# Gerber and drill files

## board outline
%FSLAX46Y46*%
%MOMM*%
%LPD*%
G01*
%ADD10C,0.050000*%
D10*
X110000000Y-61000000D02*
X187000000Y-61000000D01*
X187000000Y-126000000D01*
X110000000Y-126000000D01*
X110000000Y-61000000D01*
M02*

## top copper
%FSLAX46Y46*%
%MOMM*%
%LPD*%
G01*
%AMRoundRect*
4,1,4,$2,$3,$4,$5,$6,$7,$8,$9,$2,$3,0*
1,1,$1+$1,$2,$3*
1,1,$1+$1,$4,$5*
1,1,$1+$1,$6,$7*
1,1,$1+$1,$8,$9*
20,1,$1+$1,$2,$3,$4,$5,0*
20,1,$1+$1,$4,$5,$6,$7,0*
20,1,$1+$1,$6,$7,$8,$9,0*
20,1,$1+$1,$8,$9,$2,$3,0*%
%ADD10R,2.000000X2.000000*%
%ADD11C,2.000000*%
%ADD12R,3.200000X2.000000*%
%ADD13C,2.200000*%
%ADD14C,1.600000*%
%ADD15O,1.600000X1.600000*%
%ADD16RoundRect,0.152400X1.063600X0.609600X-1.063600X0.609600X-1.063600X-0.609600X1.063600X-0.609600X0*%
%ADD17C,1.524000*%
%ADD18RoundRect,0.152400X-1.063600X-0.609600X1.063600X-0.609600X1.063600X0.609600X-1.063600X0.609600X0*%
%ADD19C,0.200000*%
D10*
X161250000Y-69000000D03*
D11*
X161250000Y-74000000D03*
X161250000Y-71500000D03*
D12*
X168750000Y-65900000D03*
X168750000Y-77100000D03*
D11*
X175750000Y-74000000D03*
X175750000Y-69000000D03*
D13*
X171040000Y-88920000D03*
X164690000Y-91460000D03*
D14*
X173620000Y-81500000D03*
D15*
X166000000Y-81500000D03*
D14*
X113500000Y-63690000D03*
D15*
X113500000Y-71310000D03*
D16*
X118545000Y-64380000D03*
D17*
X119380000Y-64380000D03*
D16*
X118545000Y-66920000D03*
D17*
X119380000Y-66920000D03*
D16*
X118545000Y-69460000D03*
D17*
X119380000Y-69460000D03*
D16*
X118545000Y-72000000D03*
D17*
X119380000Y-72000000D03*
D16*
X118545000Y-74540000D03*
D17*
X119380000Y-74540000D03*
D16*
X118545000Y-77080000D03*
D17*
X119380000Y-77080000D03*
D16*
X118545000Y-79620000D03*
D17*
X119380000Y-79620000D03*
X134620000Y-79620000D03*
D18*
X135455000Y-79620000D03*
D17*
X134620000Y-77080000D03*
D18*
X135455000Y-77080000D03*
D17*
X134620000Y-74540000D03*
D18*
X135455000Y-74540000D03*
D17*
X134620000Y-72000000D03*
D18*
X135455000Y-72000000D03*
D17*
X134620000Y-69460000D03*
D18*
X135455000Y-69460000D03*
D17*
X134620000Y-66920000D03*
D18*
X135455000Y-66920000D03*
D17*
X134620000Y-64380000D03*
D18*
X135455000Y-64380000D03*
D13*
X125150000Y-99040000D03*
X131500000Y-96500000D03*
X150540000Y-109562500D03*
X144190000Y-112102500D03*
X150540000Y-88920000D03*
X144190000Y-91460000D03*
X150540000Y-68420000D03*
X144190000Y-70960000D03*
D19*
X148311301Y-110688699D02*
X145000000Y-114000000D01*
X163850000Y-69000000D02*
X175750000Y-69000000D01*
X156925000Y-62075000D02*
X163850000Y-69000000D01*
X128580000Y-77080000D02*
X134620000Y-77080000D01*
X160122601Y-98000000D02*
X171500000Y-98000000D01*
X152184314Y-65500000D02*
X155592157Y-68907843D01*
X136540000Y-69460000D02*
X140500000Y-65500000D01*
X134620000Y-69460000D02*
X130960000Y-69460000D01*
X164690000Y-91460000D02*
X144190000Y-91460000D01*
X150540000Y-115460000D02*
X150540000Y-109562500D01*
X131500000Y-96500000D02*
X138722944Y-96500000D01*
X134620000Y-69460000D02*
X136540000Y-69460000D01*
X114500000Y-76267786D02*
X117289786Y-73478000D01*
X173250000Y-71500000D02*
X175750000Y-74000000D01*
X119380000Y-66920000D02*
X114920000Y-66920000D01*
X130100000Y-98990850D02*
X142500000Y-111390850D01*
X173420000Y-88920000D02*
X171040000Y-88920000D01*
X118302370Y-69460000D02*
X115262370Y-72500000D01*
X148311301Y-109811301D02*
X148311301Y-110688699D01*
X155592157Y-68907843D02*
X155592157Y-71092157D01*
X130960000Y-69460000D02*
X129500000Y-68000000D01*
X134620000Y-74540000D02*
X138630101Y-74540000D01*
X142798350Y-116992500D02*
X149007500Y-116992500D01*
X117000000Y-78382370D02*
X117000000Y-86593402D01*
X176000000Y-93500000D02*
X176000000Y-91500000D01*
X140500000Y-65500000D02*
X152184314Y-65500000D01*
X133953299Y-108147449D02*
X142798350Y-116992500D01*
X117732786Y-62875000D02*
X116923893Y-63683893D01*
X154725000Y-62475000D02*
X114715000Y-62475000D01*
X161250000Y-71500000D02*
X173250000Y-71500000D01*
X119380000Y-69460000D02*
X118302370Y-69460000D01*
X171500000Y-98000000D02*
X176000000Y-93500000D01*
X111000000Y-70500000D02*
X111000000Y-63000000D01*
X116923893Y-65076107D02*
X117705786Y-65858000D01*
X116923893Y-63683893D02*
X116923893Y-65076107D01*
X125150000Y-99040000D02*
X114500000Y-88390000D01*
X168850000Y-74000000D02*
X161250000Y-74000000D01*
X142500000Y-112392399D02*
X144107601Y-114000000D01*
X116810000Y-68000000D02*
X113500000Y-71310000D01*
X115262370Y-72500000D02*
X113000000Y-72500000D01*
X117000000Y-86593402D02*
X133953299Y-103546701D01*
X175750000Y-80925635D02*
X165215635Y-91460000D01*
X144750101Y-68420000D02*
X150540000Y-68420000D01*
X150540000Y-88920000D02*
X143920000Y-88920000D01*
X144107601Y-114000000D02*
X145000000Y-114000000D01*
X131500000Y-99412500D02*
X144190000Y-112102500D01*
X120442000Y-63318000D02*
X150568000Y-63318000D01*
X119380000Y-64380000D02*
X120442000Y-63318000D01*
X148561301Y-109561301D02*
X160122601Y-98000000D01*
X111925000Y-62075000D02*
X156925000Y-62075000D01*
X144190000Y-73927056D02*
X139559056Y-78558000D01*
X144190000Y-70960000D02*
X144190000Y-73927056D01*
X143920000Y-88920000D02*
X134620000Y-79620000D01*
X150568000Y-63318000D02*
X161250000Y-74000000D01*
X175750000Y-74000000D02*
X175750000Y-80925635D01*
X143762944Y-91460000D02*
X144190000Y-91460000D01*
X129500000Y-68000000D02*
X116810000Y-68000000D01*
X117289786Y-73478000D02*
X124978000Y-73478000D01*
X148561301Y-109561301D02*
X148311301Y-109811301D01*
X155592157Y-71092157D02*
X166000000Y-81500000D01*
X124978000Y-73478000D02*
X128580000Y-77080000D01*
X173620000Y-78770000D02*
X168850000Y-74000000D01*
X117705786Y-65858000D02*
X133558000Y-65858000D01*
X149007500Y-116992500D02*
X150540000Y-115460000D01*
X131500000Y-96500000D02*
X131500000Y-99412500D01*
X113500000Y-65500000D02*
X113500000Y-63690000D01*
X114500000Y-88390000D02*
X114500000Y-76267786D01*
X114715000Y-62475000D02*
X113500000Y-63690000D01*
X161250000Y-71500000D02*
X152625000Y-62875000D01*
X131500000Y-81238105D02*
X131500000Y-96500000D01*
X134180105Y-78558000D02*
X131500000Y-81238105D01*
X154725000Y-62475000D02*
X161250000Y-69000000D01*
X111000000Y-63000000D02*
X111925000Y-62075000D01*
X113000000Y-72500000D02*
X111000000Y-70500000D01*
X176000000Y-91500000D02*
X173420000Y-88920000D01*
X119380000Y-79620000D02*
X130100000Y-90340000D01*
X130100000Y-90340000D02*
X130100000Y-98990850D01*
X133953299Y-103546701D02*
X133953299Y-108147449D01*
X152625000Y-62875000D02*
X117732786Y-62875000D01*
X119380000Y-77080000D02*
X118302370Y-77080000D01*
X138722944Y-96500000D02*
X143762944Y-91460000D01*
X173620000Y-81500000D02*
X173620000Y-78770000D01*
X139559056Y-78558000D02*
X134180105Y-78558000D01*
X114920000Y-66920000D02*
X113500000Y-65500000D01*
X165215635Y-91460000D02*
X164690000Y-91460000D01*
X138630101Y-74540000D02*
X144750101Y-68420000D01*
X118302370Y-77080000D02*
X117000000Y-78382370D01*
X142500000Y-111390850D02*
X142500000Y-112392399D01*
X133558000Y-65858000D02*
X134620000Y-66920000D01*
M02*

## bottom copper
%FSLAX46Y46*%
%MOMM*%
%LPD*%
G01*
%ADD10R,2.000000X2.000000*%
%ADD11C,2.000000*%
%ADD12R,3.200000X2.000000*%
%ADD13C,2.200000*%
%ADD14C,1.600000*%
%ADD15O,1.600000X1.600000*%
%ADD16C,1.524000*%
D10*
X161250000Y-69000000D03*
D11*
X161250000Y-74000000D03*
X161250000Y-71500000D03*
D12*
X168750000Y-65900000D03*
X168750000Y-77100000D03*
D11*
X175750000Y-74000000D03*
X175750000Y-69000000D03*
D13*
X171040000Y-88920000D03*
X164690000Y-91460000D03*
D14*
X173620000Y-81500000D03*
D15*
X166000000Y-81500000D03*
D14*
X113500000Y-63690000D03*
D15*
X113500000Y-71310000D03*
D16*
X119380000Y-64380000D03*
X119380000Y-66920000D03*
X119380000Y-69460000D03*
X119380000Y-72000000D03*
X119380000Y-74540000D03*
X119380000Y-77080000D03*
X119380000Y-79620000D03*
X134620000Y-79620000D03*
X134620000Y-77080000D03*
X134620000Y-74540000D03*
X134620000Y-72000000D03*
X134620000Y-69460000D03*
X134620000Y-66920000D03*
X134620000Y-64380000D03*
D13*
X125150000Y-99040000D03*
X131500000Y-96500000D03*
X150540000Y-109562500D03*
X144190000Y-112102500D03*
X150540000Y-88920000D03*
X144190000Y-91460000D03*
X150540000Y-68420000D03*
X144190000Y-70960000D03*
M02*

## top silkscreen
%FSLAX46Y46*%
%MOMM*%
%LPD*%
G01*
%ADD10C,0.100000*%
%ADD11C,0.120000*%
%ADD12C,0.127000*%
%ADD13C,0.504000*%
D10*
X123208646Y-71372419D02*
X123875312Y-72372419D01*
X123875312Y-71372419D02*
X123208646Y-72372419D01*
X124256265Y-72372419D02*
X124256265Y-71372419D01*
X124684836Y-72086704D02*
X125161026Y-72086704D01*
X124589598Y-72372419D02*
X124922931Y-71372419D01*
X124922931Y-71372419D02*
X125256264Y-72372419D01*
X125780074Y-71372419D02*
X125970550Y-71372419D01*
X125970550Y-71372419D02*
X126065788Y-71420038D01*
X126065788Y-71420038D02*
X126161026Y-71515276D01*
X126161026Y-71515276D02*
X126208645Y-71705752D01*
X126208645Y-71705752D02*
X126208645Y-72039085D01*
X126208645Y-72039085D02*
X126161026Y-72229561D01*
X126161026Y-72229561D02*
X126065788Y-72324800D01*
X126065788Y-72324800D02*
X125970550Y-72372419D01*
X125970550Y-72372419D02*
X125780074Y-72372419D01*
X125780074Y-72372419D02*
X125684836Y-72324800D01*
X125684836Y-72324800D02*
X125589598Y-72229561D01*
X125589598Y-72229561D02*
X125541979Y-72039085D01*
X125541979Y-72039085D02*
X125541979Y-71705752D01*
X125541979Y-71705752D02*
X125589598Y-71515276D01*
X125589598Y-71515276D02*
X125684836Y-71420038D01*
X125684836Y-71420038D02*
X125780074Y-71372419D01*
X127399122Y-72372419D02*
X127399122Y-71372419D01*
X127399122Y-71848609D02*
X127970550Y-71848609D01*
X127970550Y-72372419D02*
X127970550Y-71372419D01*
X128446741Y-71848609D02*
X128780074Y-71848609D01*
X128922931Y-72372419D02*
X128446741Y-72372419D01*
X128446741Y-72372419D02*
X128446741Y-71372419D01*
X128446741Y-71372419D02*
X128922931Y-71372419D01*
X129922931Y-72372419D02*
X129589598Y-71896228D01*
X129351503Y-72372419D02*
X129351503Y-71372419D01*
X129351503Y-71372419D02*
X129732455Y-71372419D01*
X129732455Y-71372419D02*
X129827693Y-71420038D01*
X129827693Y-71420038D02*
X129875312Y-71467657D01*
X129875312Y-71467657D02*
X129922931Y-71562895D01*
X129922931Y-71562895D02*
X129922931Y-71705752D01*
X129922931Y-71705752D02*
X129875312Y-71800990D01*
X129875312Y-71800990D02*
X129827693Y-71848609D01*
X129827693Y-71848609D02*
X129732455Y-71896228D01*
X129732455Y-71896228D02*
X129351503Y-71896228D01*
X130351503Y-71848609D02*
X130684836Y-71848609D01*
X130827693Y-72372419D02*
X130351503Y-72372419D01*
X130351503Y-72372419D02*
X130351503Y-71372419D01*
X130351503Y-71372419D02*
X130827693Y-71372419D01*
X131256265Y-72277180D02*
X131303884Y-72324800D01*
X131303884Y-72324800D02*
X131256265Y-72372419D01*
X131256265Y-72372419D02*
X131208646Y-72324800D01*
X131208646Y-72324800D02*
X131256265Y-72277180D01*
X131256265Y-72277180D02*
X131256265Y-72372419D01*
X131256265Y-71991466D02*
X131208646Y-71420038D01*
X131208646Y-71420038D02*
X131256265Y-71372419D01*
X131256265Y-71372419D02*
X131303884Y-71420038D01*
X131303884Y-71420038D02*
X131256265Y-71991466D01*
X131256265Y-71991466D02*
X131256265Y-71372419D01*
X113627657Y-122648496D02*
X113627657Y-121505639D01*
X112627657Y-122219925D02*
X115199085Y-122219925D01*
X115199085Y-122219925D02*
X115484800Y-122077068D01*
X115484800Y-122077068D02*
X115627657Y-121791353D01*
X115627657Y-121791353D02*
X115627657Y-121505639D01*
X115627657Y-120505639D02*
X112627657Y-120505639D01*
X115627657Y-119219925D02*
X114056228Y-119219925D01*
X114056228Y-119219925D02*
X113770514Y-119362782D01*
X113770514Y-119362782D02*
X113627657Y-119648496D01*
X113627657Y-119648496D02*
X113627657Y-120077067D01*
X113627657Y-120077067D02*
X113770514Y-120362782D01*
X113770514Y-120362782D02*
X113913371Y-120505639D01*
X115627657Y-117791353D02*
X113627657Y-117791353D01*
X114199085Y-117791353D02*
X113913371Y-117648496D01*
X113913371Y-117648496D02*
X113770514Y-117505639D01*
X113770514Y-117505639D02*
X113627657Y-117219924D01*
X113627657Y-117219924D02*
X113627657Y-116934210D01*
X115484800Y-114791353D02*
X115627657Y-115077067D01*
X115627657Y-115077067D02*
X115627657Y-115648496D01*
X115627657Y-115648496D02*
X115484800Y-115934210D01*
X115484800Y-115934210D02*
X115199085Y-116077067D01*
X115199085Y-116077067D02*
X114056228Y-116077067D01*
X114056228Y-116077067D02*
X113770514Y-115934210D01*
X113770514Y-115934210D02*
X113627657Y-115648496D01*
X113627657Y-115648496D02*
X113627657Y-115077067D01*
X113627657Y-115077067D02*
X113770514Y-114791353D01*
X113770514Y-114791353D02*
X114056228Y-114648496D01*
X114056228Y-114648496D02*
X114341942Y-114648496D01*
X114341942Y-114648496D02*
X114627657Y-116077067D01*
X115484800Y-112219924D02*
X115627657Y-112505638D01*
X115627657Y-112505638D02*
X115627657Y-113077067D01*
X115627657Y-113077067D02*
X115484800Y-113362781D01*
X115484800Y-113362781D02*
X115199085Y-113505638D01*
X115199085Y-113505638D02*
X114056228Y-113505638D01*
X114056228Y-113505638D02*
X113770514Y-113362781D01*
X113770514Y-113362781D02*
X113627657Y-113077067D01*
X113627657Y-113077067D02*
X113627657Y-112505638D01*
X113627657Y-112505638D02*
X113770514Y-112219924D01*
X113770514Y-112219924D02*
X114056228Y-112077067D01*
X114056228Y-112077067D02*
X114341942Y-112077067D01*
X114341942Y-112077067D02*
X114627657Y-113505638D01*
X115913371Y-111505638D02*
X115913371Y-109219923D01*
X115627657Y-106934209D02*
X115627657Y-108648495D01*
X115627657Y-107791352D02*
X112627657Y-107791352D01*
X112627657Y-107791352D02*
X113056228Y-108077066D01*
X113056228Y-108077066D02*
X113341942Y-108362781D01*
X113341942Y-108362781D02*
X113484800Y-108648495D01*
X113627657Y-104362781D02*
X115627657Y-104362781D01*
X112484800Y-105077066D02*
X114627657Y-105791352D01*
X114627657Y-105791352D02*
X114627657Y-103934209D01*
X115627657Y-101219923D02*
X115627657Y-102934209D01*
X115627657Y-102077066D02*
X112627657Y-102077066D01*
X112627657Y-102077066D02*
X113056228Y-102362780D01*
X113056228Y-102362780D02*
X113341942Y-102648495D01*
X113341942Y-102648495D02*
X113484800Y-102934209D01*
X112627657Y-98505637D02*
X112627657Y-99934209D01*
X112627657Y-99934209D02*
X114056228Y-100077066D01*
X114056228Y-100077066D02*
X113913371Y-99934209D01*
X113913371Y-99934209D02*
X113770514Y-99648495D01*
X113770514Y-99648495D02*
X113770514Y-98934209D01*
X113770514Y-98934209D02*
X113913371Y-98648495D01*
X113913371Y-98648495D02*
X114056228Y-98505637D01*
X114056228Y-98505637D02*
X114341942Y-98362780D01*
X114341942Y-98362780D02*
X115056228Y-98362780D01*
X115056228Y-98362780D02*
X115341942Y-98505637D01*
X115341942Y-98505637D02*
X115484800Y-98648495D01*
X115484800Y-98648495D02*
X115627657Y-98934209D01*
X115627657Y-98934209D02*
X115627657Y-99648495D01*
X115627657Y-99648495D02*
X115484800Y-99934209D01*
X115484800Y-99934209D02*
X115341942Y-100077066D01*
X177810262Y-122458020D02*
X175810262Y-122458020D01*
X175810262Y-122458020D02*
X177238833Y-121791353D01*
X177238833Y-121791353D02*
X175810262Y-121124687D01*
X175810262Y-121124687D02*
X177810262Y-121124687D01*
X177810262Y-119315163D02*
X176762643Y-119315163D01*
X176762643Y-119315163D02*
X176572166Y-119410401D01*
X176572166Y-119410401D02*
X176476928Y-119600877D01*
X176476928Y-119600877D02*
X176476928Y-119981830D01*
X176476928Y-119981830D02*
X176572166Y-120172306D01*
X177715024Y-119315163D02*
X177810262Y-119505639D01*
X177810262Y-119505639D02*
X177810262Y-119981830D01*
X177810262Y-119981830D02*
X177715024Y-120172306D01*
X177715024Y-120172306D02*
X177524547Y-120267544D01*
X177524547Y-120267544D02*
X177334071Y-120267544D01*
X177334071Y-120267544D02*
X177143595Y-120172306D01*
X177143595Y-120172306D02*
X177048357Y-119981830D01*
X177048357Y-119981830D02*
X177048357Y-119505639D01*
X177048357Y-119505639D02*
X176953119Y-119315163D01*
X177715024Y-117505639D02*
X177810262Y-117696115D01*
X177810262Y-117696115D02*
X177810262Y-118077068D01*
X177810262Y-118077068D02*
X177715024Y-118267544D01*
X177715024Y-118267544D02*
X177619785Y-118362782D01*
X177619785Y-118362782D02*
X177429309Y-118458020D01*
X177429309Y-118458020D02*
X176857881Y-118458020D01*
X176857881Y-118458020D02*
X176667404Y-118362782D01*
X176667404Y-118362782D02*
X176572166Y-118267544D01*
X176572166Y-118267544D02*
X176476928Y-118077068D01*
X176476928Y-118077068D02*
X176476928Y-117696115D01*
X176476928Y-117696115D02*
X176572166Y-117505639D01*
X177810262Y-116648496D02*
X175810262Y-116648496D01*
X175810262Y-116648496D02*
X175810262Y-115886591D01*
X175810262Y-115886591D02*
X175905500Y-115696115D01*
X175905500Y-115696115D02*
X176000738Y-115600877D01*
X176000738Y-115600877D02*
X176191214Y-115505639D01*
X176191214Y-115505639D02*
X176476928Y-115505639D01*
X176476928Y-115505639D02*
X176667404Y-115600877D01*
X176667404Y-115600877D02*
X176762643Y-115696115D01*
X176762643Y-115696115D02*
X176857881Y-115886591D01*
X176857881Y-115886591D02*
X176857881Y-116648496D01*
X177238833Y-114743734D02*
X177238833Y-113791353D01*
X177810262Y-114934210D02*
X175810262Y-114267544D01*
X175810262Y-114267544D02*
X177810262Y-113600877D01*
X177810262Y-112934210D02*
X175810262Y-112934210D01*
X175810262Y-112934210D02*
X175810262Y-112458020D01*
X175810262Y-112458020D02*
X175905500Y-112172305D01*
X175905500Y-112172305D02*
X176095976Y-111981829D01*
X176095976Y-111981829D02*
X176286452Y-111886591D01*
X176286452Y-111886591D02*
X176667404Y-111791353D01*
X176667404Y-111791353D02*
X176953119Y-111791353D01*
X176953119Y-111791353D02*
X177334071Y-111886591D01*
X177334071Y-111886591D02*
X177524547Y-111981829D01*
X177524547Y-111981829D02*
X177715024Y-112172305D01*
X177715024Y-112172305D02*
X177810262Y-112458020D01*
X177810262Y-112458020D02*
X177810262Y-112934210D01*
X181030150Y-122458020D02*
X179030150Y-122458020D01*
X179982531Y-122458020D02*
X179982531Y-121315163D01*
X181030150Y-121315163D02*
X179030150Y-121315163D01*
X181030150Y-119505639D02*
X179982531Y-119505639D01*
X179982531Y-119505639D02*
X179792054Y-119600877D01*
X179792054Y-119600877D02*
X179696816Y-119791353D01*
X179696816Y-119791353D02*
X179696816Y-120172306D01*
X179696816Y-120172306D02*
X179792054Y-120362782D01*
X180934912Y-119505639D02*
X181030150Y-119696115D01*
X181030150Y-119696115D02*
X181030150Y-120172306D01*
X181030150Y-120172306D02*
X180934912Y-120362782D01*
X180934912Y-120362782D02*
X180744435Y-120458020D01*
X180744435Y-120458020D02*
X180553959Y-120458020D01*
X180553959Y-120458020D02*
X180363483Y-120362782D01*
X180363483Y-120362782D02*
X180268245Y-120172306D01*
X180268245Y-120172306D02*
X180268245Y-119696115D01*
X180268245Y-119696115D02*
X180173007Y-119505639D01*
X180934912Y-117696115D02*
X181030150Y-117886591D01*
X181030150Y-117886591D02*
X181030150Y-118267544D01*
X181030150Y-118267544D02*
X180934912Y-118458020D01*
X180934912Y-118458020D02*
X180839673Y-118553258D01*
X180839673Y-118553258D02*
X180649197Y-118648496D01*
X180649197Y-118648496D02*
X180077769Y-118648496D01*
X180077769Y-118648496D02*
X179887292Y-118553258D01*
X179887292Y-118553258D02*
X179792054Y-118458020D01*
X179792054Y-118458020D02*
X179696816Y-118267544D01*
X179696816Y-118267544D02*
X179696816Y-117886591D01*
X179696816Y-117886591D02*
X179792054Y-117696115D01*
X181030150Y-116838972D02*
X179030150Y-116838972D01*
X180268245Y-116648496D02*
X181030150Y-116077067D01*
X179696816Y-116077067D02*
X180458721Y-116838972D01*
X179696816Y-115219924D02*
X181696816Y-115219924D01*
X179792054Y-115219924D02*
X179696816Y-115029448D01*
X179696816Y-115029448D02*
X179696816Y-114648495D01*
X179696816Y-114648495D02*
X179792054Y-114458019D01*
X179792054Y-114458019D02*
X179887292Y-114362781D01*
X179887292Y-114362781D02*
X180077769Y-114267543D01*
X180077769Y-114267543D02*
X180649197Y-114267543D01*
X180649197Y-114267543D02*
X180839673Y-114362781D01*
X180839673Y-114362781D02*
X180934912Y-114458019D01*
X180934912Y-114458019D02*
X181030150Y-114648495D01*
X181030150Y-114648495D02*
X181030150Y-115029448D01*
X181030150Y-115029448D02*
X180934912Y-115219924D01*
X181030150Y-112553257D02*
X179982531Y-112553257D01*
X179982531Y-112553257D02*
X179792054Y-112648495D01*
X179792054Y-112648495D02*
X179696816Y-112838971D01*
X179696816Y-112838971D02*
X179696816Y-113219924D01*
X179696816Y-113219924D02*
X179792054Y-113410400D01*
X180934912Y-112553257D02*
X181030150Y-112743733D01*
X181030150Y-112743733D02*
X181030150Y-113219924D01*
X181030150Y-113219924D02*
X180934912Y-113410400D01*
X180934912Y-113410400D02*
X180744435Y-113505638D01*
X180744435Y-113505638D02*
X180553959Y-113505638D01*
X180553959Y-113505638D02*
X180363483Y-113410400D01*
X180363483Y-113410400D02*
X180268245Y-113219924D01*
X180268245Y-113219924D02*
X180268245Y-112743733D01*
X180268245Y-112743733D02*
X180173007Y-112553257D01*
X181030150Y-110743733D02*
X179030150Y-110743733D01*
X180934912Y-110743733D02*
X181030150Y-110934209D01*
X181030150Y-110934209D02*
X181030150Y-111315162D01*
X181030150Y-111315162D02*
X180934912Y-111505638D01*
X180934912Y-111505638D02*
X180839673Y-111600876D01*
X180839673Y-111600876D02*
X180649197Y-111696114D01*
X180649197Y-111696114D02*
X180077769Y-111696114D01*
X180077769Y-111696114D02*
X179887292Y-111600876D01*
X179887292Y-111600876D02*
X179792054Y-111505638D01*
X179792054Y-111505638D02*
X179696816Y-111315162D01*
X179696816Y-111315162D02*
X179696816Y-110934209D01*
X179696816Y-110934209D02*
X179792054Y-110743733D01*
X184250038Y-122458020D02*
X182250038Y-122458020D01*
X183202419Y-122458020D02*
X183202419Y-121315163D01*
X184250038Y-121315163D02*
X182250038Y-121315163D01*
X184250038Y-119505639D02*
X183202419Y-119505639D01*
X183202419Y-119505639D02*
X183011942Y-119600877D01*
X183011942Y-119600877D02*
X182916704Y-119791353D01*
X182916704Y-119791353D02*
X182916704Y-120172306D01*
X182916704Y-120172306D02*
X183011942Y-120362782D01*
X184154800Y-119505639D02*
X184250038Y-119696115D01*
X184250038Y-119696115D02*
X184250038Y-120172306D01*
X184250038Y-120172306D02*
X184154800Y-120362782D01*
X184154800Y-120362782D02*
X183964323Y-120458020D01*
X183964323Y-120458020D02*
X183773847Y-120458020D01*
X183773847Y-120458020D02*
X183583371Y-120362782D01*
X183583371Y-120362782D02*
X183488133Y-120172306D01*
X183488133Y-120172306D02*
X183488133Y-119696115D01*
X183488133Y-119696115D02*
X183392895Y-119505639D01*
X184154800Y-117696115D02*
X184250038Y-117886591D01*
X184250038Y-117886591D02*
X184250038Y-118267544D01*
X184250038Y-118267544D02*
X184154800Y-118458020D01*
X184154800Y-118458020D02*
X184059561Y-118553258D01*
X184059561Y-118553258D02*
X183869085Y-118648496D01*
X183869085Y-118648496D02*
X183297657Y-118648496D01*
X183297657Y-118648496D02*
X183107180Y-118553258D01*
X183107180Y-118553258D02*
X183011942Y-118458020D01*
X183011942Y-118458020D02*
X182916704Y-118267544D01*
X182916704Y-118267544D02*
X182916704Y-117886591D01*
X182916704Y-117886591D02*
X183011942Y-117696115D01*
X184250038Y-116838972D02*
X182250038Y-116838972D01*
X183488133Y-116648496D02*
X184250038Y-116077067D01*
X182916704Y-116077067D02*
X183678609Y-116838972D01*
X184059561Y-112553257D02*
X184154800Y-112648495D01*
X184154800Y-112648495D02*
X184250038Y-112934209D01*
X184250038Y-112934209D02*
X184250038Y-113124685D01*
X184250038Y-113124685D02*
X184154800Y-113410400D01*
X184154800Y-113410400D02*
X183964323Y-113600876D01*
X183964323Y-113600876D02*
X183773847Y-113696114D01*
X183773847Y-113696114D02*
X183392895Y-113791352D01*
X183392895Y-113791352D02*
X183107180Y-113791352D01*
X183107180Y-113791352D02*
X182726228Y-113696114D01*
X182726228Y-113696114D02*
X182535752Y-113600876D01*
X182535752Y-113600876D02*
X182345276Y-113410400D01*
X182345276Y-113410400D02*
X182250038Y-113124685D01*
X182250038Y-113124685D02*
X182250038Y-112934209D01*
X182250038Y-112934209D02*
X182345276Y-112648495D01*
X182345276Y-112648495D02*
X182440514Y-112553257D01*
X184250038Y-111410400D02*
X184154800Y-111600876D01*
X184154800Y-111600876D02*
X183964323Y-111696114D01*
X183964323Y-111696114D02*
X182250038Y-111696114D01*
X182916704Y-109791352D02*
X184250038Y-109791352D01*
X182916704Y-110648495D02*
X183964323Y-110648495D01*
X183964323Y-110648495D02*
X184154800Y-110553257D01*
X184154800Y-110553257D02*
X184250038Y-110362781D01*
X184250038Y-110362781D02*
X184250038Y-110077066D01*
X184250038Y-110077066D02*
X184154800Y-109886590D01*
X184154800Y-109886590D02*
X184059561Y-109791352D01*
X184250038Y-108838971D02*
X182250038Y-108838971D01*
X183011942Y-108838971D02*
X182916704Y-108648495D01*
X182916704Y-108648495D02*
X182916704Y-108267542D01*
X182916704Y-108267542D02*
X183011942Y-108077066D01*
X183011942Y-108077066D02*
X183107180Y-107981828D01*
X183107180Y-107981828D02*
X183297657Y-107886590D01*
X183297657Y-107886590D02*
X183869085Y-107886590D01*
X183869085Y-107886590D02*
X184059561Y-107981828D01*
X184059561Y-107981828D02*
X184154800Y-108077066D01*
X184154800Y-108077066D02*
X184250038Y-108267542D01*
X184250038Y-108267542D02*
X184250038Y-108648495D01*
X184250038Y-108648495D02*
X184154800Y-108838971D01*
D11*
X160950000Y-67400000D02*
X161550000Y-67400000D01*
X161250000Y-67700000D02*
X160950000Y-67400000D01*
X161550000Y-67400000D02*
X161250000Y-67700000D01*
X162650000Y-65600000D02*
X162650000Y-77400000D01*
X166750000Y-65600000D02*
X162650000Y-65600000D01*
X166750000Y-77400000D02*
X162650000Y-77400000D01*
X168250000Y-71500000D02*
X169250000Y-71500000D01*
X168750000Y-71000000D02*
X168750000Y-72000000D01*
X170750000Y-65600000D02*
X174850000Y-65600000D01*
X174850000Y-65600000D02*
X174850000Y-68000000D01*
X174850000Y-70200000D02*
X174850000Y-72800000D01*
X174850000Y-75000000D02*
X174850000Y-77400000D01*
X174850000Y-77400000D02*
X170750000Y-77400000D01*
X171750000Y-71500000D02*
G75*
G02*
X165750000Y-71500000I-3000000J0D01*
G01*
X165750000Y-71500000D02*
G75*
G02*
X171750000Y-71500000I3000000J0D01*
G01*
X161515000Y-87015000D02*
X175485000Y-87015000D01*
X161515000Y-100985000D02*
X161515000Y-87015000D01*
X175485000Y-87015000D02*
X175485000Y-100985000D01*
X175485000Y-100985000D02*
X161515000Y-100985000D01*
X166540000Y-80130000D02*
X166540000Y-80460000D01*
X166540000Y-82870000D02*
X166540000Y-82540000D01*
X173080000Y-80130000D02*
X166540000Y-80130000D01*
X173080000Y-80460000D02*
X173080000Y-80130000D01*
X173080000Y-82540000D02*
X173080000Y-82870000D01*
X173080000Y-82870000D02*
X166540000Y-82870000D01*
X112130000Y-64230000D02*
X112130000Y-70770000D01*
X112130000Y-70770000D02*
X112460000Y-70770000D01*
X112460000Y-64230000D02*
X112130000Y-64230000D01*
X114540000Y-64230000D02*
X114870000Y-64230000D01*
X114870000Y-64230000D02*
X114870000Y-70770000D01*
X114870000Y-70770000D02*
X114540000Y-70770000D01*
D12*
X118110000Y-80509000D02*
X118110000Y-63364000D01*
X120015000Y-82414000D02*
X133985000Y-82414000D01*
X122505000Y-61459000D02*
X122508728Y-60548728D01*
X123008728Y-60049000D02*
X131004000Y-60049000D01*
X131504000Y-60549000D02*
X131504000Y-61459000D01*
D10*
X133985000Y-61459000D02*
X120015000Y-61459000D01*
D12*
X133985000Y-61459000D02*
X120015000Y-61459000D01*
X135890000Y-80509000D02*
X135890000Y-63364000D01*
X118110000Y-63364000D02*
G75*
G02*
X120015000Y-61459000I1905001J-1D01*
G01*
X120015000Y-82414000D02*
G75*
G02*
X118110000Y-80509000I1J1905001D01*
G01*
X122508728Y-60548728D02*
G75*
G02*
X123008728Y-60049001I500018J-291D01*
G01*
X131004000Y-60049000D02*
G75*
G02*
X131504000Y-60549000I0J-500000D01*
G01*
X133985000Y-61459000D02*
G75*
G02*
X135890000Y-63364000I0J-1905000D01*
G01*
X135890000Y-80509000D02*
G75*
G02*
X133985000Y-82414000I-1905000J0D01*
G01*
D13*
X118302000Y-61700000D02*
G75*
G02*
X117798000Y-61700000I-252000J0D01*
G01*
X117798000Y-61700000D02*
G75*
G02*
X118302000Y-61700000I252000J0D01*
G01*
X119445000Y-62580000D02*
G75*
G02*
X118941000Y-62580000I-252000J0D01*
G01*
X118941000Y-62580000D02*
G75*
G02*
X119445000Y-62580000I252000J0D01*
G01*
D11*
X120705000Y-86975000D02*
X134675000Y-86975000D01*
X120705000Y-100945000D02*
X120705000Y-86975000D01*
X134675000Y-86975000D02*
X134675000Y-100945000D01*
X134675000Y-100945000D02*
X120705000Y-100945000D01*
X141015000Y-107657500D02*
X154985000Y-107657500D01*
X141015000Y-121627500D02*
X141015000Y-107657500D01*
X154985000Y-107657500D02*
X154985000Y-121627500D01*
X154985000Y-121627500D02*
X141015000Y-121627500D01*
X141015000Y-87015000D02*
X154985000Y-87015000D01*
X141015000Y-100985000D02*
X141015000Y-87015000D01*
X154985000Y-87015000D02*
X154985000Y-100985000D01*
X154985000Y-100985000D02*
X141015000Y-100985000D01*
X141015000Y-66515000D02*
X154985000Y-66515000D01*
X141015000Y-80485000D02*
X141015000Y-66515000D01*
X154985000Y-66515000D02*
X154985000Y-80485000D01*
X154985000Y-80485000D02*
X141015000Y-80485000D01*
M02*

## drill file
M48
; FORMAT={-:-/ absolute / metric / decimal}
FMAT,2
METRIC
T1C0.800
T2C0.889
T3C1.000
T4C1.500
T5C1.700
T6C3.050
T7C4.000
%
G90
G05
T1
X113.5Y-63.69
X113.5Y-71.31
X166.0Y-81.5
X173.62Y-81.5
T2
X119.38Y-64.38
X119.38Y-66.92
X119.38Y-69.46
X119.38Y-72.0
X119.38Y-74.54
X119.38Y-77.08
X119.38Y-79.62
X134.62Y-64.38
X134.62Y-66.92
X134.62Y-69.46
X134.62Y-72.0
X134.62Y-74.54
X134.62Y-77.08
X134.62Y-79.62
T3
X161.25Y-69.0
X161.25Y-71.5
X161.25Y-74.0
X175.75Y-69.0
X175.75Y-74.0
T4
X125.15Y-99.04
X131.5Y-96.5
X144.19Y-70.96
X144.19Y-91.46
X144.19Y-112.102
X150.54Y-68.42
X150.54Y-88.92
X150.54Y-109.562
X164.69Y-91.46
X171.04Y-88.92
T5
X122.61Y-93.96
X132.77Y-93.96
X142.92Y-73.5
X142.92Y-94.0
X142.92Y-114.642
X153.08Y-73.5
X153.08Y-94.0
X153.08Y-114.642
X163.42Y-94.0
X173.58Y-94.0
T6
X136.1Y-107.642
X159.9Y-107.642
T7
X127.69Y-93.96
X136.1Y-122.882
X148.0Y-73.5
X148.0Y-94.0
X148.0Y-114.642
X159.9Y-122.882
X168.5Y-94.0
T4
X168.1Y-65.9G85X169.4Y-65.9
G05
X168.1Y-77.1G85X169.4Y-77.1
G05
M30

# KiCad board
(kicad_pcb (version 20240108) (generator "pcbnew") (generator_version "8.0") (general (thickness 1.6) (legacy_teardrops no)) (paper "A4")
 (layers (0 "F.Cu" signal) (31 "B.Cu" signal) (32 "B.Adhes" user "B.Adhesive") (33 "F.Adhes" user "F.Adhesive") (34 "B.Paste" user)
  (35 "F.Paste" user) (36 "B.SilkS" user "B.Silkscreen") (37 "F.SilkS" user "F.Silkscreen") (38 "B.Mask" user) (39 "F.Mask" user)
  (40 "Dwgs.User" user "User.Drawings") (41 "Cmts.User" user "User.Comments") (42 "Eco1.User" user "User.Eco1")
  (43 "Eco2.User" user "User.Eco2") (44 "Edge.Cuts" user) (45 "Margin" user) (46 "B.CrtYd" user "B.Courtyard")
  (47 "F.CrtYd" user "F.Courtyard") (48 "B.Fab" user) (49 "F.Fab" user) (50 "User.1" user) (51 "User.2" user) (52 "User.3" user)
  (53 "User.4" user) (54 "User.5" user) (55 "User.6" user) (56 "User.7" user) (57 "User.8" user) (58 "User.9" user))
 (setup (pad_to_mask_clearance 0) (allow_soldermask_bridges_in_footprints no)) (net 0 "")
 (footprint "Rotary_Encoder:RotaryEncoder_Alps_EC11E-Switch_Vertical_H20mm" (layer "F.Cu") (at 161.25 69)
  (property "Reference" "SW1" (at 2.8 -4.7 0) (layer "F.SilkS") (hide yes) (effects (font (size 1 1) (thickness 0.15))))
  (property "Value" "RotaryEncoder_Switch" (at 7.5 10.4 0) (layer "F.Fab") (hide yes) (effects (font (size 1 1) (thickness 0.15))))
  (fp_line (start -0.3 -1.6) (end 0.3 -1.6) (stroke (width 0.12) (type solid)) (layer "F.SilkS"))
  (fp_line (start 0 -1.3) (end -0.3 -1.6) (stroke (width 0.12) (type solid)) (layer "F.SilkS"))
  (fp_line (start 0.3 -1.6) (end 0 -1.3) (stroke (width 0.12) (type solid)) (layer "F.SilkS"))
  (fp_line (start 1.4 -3.4) (end 1.4 8.4) (stroke (width 0.12) (type solid)) (layer "F.SilkS"))
  (fp_line (start 5.5 -3.4) (end 1.4 -3.4) (stroke (width 0.12) (type solid)) (layer "F.SilkS"))
  (fp_line (start 5.5 8.4) (end 1.4 8.4) (stroke (width 0.12) (type solid)) (layer "F.SilkS"))
  (fp_line (start 7 2.5) (end 8 2.5) (stroke (width 0.12) (type solid)) (layer "F.SilkS"))
  (fp_line (start 7.5 2) (end 7.5 3) (stroke (width 0.12) (type solid)) (layer "F.SilkS"))
  (fp_line (start 9.5 -3.4) (end 13.6 -3.4) (stroke (width 0.12) (type solid)) (layer "F.SilkS"))
  (fp_line (start 13.6 -3.4) (end 13.6 -1) (stroke (width 0.12) (type solid)) (layer "F.SilkS"))
  (fp_line (start 13.6 1.2) (end 13.6 3.8) (stroke (width 0.12) (type solid)) (layer "F.SilkS"))
  (fp_line (start 13.6 6) (end 13.6 8.4) (stroke (width 0.12) (type solid)) (layer "F.SilkS"))
  (fp_line (start 13.6 8.4) (end 9.5 8.4) (stroke (width 0.12) (type solid)) (layer "F.SilkS"))
  (fp_circle (center 7.5 2.5) (end 10.5 2.5) (stroke (width 0.12) (type solid)) (fill none) (layer "F.SilkS"))
  (pad "A" thru_hole rect (at 0 0) (size 2 2) (drill 1) (layers "*.Cu" "*.Mask") (remove_unused_layers no))
  (pad "B" thru_hole circle (at 0 5) (size 2 2) (drill 1) (layers "*.Cu" "*.Mask") (remove_unused_layers no))
  (pad "C" thru_hole circle (at 0 2.5) (size 2 2) (drill 1) (layers "*.Cu" "*.Mask") (remove_unused_layers no))
  (pad "MP" thru_hole rect (at 7.5 -3.1) (size 3.2 2) (drill oval 2.8 1.5) (layers "*.Cu" "*.Mask") (remove_unused_layers no))
  (pad "MP" thru_hole rect (at 7.5 8.1) (size 3.2 2) (drill oval 2.8 1.5) (layers "*.Cu" "*.Mask") (remove_unused_layers no))
  (pad "S1" thru_hole circle (at 14.5 5) (size 2 2) (drill 1) (layers "*.Cu" "*.Mask") (remove_unused_layers no))
  (pad "S2" thru_hole circle (at 14.5 0) (size 2 2) (drill 1) (layers "*.Cu" "*.Mask") (remove_unused_layers no)))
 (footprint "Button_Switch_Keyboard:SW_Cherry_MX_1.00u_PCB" (layer "F.Cu") (at 171.04 88.92)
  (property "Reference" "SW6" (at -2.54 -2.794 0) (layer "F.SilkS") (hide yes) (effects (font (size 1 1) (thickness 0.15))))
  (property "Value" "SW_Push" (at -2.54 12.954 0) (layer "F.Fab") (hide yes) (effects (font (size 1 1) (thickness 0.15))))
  (fp_line (start -9.525 -1.905) (end 4.445 -1.905) (stroke (width 0.12) (type solid)) (layer "F.SilkS"))
  (fp_line (start -9.525 12.065) (end -9.525 -1.905) (stroke (width 0.12) (type solid)) (layer "F.SilkS"))
  (fp_line (start 4.445 -1.905) (end 4.445 12.065) (stroke (width 0.12) (type solid)) (layer "F.SilkS"))
  (fp_line (start 4.445 12.065) (end -9.525 12.065) (stroke (width 0.12) (type solid)) (layer "F.SilkS"))
  (pad "" np_thru_hole circle (at -7.62 5.08) (size 1.7 1.7) (drill 1.7) (layers "*.Cu" "*.Mask"))
  (pad "" np_thru_hole circle (at -2.54 5.08) (size 4 4) (drill 4) (layers "*.Cu" "*.Mask"))
  (pad "" np_thru_hole circle (at 2.54 5.08) (size 1.7 1.7) (drill 1.7) (layers "*.Cu" "*.Mask"))
  (pad "1" thru_hole circle (at 0 0) (size 2.2 2.2) (drill 1.5) (layers "*.Cu" "*.Mask") (remove_unused_layers no))
  (pad "2" thru_hole circle (at -6.35 2.54) (size 2.2 2.2) (drill 1.5) (layers "*.Cu" "*.Mask") (remove_unused_layers no)))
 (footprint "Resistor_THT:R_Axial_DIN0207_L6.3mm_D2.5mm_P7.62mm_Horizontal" (layer "F.Cu") (at 173.62 81.5 180)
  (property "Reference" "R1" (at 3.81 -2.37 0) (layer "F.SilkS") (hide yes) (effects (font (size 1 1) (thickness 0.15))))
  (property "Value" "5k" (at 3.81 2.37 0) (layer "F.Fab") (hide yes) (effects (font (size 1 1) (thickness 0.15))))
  (fp_line (start 7.08 1.37) (end 7.08 1.04) (stroke (width 0.12) (type solid)) (layer "F.SilkS"))
  (fp_line (start 7.08 -1.37) (end 7.08 -1.04) (stroke (width 0.12) (type solid)) (layer "F.SilkS"))
  (fp_line (start 0.54 1.37) (end 7.08 1.37) (stroke (width 0.12) (type solid)) (layer "F.SilkS"))
  (fp_line (start 0.54 1.04) (end 0.54 1.37) (stroke (width 0.12) (type solid)) (layer "F.SilkS"))
  (fp_line (start 0.54 -1.04) (end 0.54 -1.37) (stroke (width 0.12) (type solid)) (layer "F.SilkS"))
  (fp_line (start 0.54 -1.37) (end 7.08 -1.37) (stroke (width 0.12) (type solid)) (layer "F.SilkS"))
  (pad "1" thru_hole circle (at 0 0 180) (size 1.6 1.6) (drill 0.8) (layers "*.Cu" "*.Mask") (remove_unused_layers no))
  (pad "2" thru_hole oval (at 7.62 0 180) (size 1.6 1.6) (drill 0.8) (layers "*.Cu" "*.Mask") (remove_unused_layers no)))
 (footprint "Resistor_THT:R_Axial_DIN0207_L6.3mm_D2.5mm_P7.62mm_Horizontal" (layer "F.Cu") (at 113.5 63.69 -90)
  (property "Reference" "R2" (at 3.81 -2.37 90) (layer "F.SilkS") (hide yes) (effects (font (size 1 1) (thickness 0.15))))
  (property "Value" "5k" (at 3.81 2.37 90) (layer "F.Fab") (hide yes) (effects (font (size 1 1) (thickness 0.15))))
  (fp_line (start 0.54 1.37) (end 7.08 1.37) (stroke (width 0.12) (type solid)) (layer "F.SilkS"))
  (fp_line (start 7.08 1.37) (end 7.08 1.04) (stroke (width 0.12) (type solid)) (layer "F.SilkS"))
  (fp_line (start 0.54 1.04) (end 0.54 1.37) (stroke (width 0.12) (type solid)) (layer "F.SilkS"))
  (fp_line (start 0.54 -1.04) (end 0.54 -1.37) (stroke (width 0.12) (type solid)) (layer "F.SilkS"))
  (fp_line (start 0.54 -1.37) (end 7.08 -1.37) (stroke (width 0.12) (type solid)) (layer "F.SilkS"))
  (fp_line (start 7.08 -1.37) (end 7.08 -1.04) (stroke (width 0.12) (type solid)) (layer "F.SilkS"))
  (pad "1" thru_hole circle (at 0 0 270) (size 1.6 1.6) (drill 0.8) (layers "*.Cu" "*.Mask") (remove_unused_layers no))
  (pad "2" thru_hole oval (at 7.62 0 270) (size 1.6 1.6) (drill 0.8) (layers "*.Cu" "*.Mask") (remove_unused_layers no)))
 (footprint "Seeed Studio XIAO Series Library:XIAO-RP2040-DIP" (layer "F.Cu") (at 127 72)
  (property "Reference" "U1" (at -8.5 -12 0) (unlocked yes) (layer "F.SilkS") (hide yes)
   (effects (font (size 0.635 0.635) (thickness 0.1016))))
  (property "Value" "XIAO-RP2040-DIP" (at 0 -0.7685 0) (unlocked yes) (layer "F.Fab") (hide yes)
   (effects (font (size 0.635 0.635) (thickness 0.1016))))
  (fp_line (start -8.89 8.509) (end -8.89 -8.636) (stroke (width 0.127) (type solid)) (layer "F.SilkS"))
  (fp_line (start -6.985 10.414) (end 6.985 10.414) (stroke (width 0.127) (type solid)) (layer "F.SilkS"))
  (fp_line (start -4.495 -10.541) (end -4.491272 -11.451272) (stroke (width 0.127) (type solid)) (layer "F.SilkS"))
  (fp_line (start -3.991272 -11.951) (end 4.004 -11.951) (stroke (width 0.127) (type solid)) (layer "F.SilkS"))
  (fp_line (start 4.504 -11.451) (end 4.504 -10.541) (stroke (width 0.127) (type solid)) (layer "F.SilkS"))
  (fp_line (start 6.985 -10.541) (end -6.985 -10.541) (stroke (width 0.1) (type solid)) (layer "F.SilkS"))
  (fp_line (start 6.985 -10.541) (end -6.985 -10.541) (stroke (width 0.127) (type solid)) (layer "F.SilkS"))
  (fp_line (start 8.89 8.509) (end 8.89 -8.636) (stroke (width 0.127) (type solid)) (layer "F.SilkS"))
  (fp_arc (start -8.89 -8.636) (mid -8.332038 -9.983038) (end -6.985 -10.541) (stroke (width 0.127) (type solid)) (layer "F.SilkS"))
  (fp_arc (start -6.985 10.414) (mid -8.332038 9.856038) (end -8.89 8.509) (stroke (width 0.127) (type solid)) (layer "F.SilkS"))
  (fp_arc (start -4.491272 -11.451272) (mid -4.344724 -11.804644) (end -3.991272 -11.951) (stroke (width 0.127) (type default))
   (layer "F.SilkS"))
  (fp_arc (start 4.004 -11.951) (mid 4.357553 -11.804553) (end 4.504 -11.451) (stroke (width 0.127) (type default)) (layer "F.SilkS"))
  (fp_arc (start 6.985 -10.541) (mid 8.332038 -9.983038) (end 8.89 -8.636) (stroke (width 0.127) (type solid)) (layer "F.SilkS"))
  (fp_arc (start 8.89 8.509) (mid 8.332038 9.856038) (end 6.985 10.414) (stroke (width 0.127) (type solid)) (layer "F.SilkS"))
  (fp_circle (center -8.95 -10.3) (end -8.95 -10.554) (stroke (width 0.5) (type solid)) (fill solid) (layer "F.SilkS"))
  (fp_circle (center -7.807 -9.42) (end -7.807 -9.674) (stroke (width 0.5) (type solid)) (fill solid) (layer "F.SilkS"))
  (pad "1" smd roundrect (at -8.455 -7.62 180) (size 2.432 1.524) (layers "F.Cu" "F.Mask") (roundrect_rratio 0.1) (thermal_bridge_angle 45))
  (pad "1" thru_hole circle (at -7.62 -7.62 180) (size 1.524 1.524) (drill 0.889) (layers "*.Cu" "*.Mask") (remove_unused_layers no))
  (pad "2" smd roundrect (at -8.455 -5.08 180) (size 2.432 1.524) (layers "F.Cu" "F.Mask") (roundrect_rratio 0.1) (thermal_bridge_angle 45))
  (pad "2" thru_hole circle (at -7.62 -5.08 180) (size 1.524 1.524) (drill 0.889) (layers "*.Cu" "*.Mask") (remove_unused_layers no))
  (pad "3" smd roundrect (at -8.455 -2.54 180) (size 2.432 1.524) (layers "F.Cu" "F.Mask") (roundrect_rratio 0.1) (thermal_bridge_angle 45))
  (pad "3" thru_hole circle (at -7.62 -2.54 180) (size 1.524 1.524) (drill 0.889) (layers "*.Cu" "*.Mask") (remove_unused_layers no))
  (pad "4" smd roundrect (at -8.455 0 180) (size 2.432 1.524) (layers "F.Cu" "F.Mask") (roundrect_rratio 0.1) (thermal_bridge_angle 45))
  (pad "4" thru_hole circle (at -7.62 0 180) (size 1.524 1.524) (drill 0.889) (layers "*.Cu" "*.Mask") (remove_unused_layers no))
  (pad "5" smd roundrect (at -8.455 2.54 180) (size 2.432 1.524) (layers "F.Cu" "F.Mask") (roundrect_rratio 0.1) (thermal_bridge_angle 45))
  (pad "5" thru_hole circle (at -7.62 2.54 180) (size 1.524 1.524) (drill 0.889) (layers "*.Cu" "*.Mask") (remove_unused_layers no))
  (pad "6" smd roundrect (at -8.455 5.08 180) (size 2.432 1.524) (layers "F.Cu" "F.Mask") (roundrect_rratio 0.1) (thermal_bridge_angle 45))
  (pad "6" thru_hole circle (at -7.62 5.08 180) (size 1.524 1.524) (drill 0.889) (layers "*.Cu" "*.Mask") (remove_unused_layers no))
  (pad "7" smd roundrect (at -8.455 7.62 180) (size 2.432 1.524) (layers "F.Cu" "F.Mask") (roundrect_rratio 0.1) (thermal_bridge_angle 45))
  (pad "7" thru_hole circle (at -7.62 7.62 180) (size 1.524 1.524) (drill 0.889) (layers "*.Cu" "*.Mask") (remove_unused_layers no))
  (pad "8" thru_hole circle (at 7.62 7.62) (size 1.524 1.524) (drill 0.889) (layers "*.Cu" "*.Mask") (remove_unused_layers no))
  (pad "8" smd roundrect (at 8.455 7.62) (size 2.432 1.524) (layers "F.Cu" "F.Mask") (roundrect_rratio 0.1) (thermal_bridge_angle 45))
  (pad "9" thru_hole circle (at 7.62 5.08) (size 1.524 1.524) (drill 0.889) (layers "*.Cu" "*.Mask") (remove_unused_layers no))
  (pad "9" smd roundrect (at 8.455 5.08) (size 2.432 1.524) (layers "F.Cu" "F.Mask") (roundrect_rratio 0.1) (thermal_bridge_angle 45))
  (pad "10" thru_hole circle (at 7.62 2.54) (size 1.524 1.524) (drill 0.889) (layers "*.Cu" "*.Mask") (remove_unused_layers no))
  (pad "10" smd roundrect (at 8.455 2.54) (size 2.432 1.524) (layers "F.Cu" "F.Mask") (roundrect_rratio 0.1) (thermal_bridge_angle 45))
  (pad "11" thru_hole circle (at 7.62 0) (size 1.524 1.524) (drill 0.889) (layers "*.Cu" "*.Mask") (remove_unused_layers no))
  (pad "11" smd roundrect (at 8.455 0) (size 2.432 1.524) (layers "F.Cu" "F.Mask") (roundrect_rratio 0.1) (thermal_bridge_angle 45))
  (pad "12" thru_hole circle (at 7.62 -2.54) (size 1.524 1.524) (drill 0.889) (layers "*.Cu" "*.Mask") (remove_unused_layers no))
  (pad "12" smd roundrect (at 8.455 -2.54) (size 2.432 1.524) (layers "F.Cu" "F.Mask") (roundrect_rratio 0.1) (thermal_bridge_angle 45))
  (pad "13" thru_hole circle (at 7.62 -5.08) (size 1.524 1.524) (drill 0.889) (layers "*.Cu" "*.Mask") (remove_unused_layers no))
  (pad "13" smd roundrect (at 8.455 -5.08) (size 2.432 1.524) (layers "F.Cu" "F.Mask") (roundrect_rratio 0.1) (thermal_bridge_angle 45))
  (pad "14" thru_hole circle (at 7.62 -7.62) (size 1.524 1.524) (drill 0.889) (layers "*.Cu" "*.Mask") (remove_unused_layers no))
  (pad "14" smd roundrect (at 8.455 -7.62) (size 2.432 1.524) (layers "F.Cu" "F.Mask") (roundrect_rratio 0.1) (thermal_bridge_angle 45)))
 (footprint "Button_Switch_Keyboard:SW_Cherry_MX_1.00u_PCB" (layer "F.Cu") (at 125.15 99.04 180)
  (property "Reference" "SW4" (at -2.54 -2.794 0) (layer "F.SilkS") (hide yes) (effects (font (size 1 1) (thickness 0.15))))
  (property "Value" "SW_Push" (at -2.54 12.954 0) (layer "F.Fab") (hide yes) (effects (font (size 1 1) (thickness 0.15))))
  (fp_line (start 4.445 12.065) (end -9.525 12.065) (stroke (width 0.12) (type solid)) (layer "F.SilkS"))
  (fp_line (start 4.445 -1.905) (end 4.445 12.065) (stroke (width 0.12) (type solid)) (layer "F.SilkS"))
  (fp_line (start -9.525 12.065) (end -9.525 -1.905) (stroke (width 0.12) (type solid)) (layer "F.SilkS"))
  (fp_line (start -9.525 -1.905) (end 4.445 -1.905) (stroke (width 0.12) (type solid)) (layer "F.SilkS"))
  (pad "" np_thru_hole circle (at -7.62 5.08 180) (size 1.7 1.7) (drill 1.7) (layers "*.Cu" "*.Mask"))
  (pad "" np_thru_hole circle (at -2.54 5.08 180) (size 4 4) (drill 4) (layers "*.Cu" "*.Mask"))
  (pad "" np_thru_hole circle (at 2.54 5.08 180) (size 1.7 1.7) (drill 1.7) (layers "*.Cu" "*.Mask"))
  (pad "1" thru_hole circle (at 0 0 180) (size 2.2 2.2) (drill 1.5) (layers "*.Cu" "*.Mask") (remove_unused_layers no))
  (pad "2" thru_hole circle (at -6.35 2.54 180) (size 2.2 2.2) (drill 1.5) (layers "*.Cu" "*.Mask") (remove_unused_layers no)))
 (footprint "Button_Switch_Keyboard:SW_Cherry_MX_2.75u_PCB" (layer "F.Cu") (at 150.54 109.5625)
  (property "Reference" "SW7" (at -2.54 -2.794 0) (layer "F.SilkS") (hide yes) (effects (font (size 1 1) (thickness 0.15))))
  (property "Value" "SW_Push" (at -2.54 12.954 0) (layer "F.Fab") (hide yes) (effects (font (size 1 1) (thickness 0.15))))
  (fp_line (start -9.525 -1.905) (end 4.445 -1.905) (stroke (width 0.12) (type solid)) (layer "F.SilkS"))
  (fp_line (start -9.525 12.065) (end -9.525 -1.905) (stroke (width 0.12) (type solid)) (layer "F.SilkS"))
  (fp_line (start 4.445 -1.905) (end 4.445 12.065) (stroke (width 0.12) (type solid)) (layer "F.SilkS"))
  (fp_line (start 4.445 12.065) (end -9.525 12.065) (stroke (width 0.12) (type solid)) (layer "F.SilkS"))
  (pad "" np_thru_hole circle (at -14.44 -1.92) (size 3.05 3.05) (drill 3.05) (layers "*.Cu" "*.Mask"))
  (pad "" np_thru_hole circle (at -14.44 13.32) (size 4 4) (drill 4) (layers "*.Cu" "*.Mask"))
  (pad "" np_thru_hole circle (at -7.62 5.08) (size 1.7 1.7) (drill 1.7) (layers "*.Cu" "*.Mask"))
  (pad "" np_thru_hole circle (at -2.54 5.08) (size 4 4) (drill 4) (layers "*.Cu" "*.Mask"))
  (pad "" np_thru_hole circle (at 2.54 5.08) (size 1.7 1.7) (drill 1.7) (layers "*.Cu" "*.Mask"))
  (pad "" np_thru_hole circle (at 9.36 -1.92) (size 3.05 3.05) (drill 3.05) (layers "*.Cu" "*.Mask"))
  (pad "" np_thru_hole circle (at 9.36 13.32) (size 4 4) (drill 4) (layers "*.Cu" "*.Mask"))
  (pad "1" thru_hole circle (at 0 0) (size 2.2 2.2) (drill 1.5) (layers "*.Cu" "*.Mask") (remove_unused_layers no))
  (pad "2" thru_hole circle (at -6.35 2.54) (size 2.2 2.2) (drill 1.5) (layers "*.Cu" "*.Mask") (remove_unused_layers no)))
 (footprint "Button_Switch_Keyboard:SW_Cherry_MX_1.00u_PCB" (layer "F.Cu") (at 150.54 88.92)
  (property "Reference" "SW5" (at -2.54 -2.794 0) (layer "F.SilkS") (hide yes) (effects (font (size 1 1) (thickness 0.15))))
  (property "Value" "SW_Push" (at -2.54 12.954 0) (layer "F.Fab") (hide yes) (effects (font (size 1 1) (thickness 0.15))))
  (fp_line (start -9.525 -1.905) (end 4.445 -1.905) (stroke (width 0.12) (type solid)) (layer "F.SilkS"))
  (fp_line (start -9.525 12.065) (end -9.525 -1.905) (stroke (width 0.12) (type solid)) (layer "F.SilkS"))
  (fp_line (start 4.445 -1.905) (end 4.445 12.065) (stroke (width 0.12) (type solid)) (layer "F.SilkS"))
  (fp_line (start 4.445 12.065) (end -9.525 12.065) (stroke (width 0.12) (type solid)) (layer "F.SilkS"))
  (pad "" np_thru_hole circle (at -7.62 5.08) (size 1.7 1.7) (drill 1.7) (layers "*.Cu" "*.Mask"))
  (pad "" np_thru_hole circle (at -2.54 5.08) (size 4 4) (drill 4) (layers "*.Cu" "*.Mask"))
  (pad "" np_thru_hole circle (at 2.54 5.08) (size 1.7 1.7) (drill 1.7) (layers "*.Cu" "*.Mask"))
  (pad "1" thru_hole circle (at 0 0) (size 2.2 2.2) (drill 1.5) (layers "*.Cu" "*.Mask") (remove_unused_layers no))
  (pad "2" thru_hole circle (at -6.35 2.54) (size 2.2 2.2) (drill 1.5) (layers "*.Cu" "*.Mask") (remove_unused_layers no)))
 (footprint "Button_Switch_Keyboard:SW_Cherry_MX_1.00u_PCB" (layer "F.Cu") (at 150.54 68.42)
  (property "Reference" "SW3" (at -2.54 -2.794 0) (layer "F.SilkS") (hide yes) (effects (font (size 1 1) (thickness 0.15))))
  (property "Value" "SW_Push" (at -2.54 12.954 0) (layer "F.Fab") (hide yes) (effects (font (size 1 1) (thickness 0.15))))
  (fp_line (start -9.525 -1.905) (end 4.445 -1.905) (stroke (width 0.12) (type solid)) (layer "F.SilkS"))
  (fp_line (start -9.525 12.065) (end -9.525 -1.905) (stroke (width 0.12) (type solid)) (layer "F.SilkS"))
  (fp_line (start 4.445 -1.905) (end 4.445 12.065) (stroke (width 0.12) (type solid)) (layer "F.SilkS"))
  (fp_line (start 4.445 12.065) (end -9.525 12.065) (stroke (width 0.12) (type solid)) (layer "F.SilkS"))
  (pad "" np_thru_hole circle (at -7.62 5.08) (size 1.7 1.7) (drill 1.7) (layers "*.Cu" "*.Mask"))
  (pad "" np_thru_hole circle (at -2.54 5.08) (size 4 4) (drill 4) (layers "*.Cu" "*.Mask"))
  (pad "" np_thru_hole circle (at 2.54 5.08) (size 1.7 1.7) (drill 1.7) (layers "*.Cu" "*.Mask"))
  (pad "1" thru_hole circle (at 0 0) (size 2.2 2.2) (drill 1.5) (layers "*.Cu" "*.Mask") (remove_unused_layers no))
  (pad "2" thru_hole circle (at -6.35 2.54) (size 2.2 2.2) (drill 1.5) (layers "*.Cu" "*.Mask") (remove_unused_layers no)))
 (gr_rect (start 110 61) (end 187 126) (stroke (width 0.05) (type default)) (fill none) (layer "Edge.Cuts"))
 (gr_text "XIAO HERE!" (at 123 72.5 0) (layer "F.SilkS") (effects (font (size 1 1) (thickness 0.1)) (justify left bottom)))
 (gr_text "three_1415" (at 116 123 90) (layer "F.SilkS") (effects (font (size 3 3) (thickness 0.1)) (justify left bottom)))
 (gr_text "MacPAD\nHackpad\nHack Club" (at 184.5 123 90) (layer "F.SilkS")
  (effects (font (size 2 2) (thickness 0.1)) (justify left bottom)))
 (segment (start 148.311301 110.688699) (end 145 114) (width 0.2) (layer "F.Cu") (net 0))
 (segment (start 163.85 69) (end 175.75 69) (width 0.2) (layer "F.Cu") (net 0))
 (segment (start 156.925 62.075) (end 163.85 69) (width 0.2) (layer "F.Cu") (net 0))
 (segment (start 128.58 77.08) (end 134.62 77.08) (width 0.2) (layer "F.Cu") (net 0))
 (segment (start 160.122601 98) (end 171.5 98) (width 0.2) (layer "F.Cu") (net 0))
 (segment (start 152.184314 65.5) (end 155.592157 68.907843) (width 0.2) (layer "F.Cu") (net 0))
 (segment (start 136.54 69.46) (end 140.5 65.5) (width 0.2) (layer "F.Cu") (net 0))
 (segment (start 134.62 69.46) (end 130.96 69.46) (width 0.2) (layer "F.Cu") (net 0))
 (segment (start 164.69 91.46) (end 144.19 91.46) (width 0.2) (layer "F.Cu") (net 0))
 (segment (start 150.54 115.46) (end 150.54 109.5625) (width 0.2) (layer "F.Cu") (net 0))
 (segment (start 131.5 96.5) (end 138.722944 96.5) (width 0.2) (layer "F.Cu") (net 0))
 (segment (start 134.62 69.46) (end 136.54 69.46) (width 0.2) (layer "F.Cu") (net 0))
 (segment (start 114.5 76.267786) (end 117.289786 73.478) (width 0.2) (layer "F.Cu") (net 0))
 (segment (start 173.25 71.5) (end 175.75 74) (width 0.2) (layer "F.Cu") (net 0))
 (segment (start 119.38 66.92) (end 114.92 66.92) (width 0.2) (layer "F.Cu") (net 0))
 (segment (start 130.1 98.99085) (end 142.5 111.39085) (width 0.2) (layer "F.Cu") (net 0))
 (segment (start 173.42 88.92) (end 171.04 88.92) (width 0.2) (layer "F.Cu") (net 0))
 (segment (start 118.30237 69.46) (end 115.26237 72.5) (width 0.2) (layer "F.Cu") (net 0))
 (segment (start 148.311301 109.811301) (end 148.311301 110.688699) (width 0.2) (layer "F.Cu") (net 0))
 (segment (start 155.592157 68.907843) (end 155.592157 71.092157) (width 0.2) (layer "F.Cu") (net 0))
 (segment (start 130.96 69.46) (end 129.5 68) (width 0.2) (layer "F.Cu") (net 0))
 (segment (start 134.62 74.54) (end 138.630101 74.54) (width 0.2) (layer "F.Cu") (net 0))
 (segment (start 142.79835 116.9925) (end 149.0075 116.9925) (width 0.2) (layer "F.Cu") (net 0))
 (segment (start 117 78.38237) (end 117 86.593402) (width 0.2) (layer "F.Cu") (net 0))
 (segment (start 176 93.5) (end 176 91.5) (width 0.2) (layer "F.Cu") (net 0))
 (segment (start 140.5 65.5) (end 152.184314 65.5) (width 0.2) (layer "F.Cu") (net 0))
 (segment (start 133.953299 108.147449) (end 142.79835 116.9925) (width 0.2) (layer "F.Cu") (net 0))
 (segment (start 117.732786 62.875) (end 116.923893 63.683893) (width 0.2) (layer "F.Cu") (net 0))
 (segment (start 154.725 62.475) (end 114.715 62.475) (width 0.2) (layer "F.Cu") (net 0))
 (segment (start 161.25 71.5) (end 173.25 71.5) (width 0.2) (layer "F.Cu") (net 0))
 (segment (start 119.38 69.46) (end 118.30237 69.46) (width 0.2) (layer "F.Cu") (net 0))
 (segment (start 171.5 98) (end 176 93.5) (width 0.2) (layer "F.Cu") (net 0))
 (segment (start 111 70.5) (end 111 63) (width 0.2) (layer "F.Cu") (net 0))
 (segment (start 116.923893 65.076107) (end 117.705786 65.858) (width 0.2) (layer "F.Cu") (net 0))
 (segment (start 116.923893 63.683893) (end 116.923893 65.076107) (width 0.2) (layer "F.Cu") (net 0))
 (segment (start 125.15 99.04) (end 114.5 88.39) (width 0.2) (layer "F.Cu") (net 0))
 (segment (start 168.85 74) (end 161.25 74) (width 0.2) (layer "F.Cu") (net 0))
 (segment (start 142.5 112.392399) (end 144.107601 114) (width 0.2) (layer "F.Cu") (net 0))
 (segment (start 116.81 68) (end 113.5 71.31) (width 0.2) (layer "F.Cu") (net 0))
 (segment (start 115.26237 72.5) (end 113 72.5) (width 0.2) (layer "F.Cu") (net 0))
 (segment (start 117 86.593402) (end 133.953299 103.546701) (width 0.2) (layer "F.Cu") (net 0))
 (segment (start 175.75 80.925635) (end 165.215635 91.46) (width 0.2) (layer "F.Cu") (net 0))
 (segment (start 144.750101 68.42) (end 150.54 68.42) (width 0.2) (layer "F.Cu") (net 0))
 (segment (start 150.54 88.92) (end 143.92 88.92) (width 0.2) (layer "F.Cu") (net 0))
 (segment (start 144.107601 114) (end 145 114) (width 0.2) (layer "F.Cu") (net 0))
 (segment (start 131.5 99.4125) (end 144.19 112.1025) (width 0.2) (layer "F.Cu") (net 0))
 (segment (start 120.442 63.318) (end 150.568 63.318) (width 0.2) (layer "F.Cu") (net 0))
 (segment (start 119.38 64.38) (end 120.442 63.318) (width 0.2) (layer "F.Cu") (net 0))
 (segment (start 148.561301 109.561301) (end 160.122601 98) (width 0.2) (layer "F.Cu") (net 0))
 (segment (start 111.925 62.075) (end 156.925 62.075) (width 0.2) (layer "F.Cu") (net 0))
 (segment (start 144.19 73.927056) (end 139.559056 78.558) (width 0.2) (layer "F.Cu") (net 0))
 (segment (start 144.19 70.96) (end 144.19 73.927056) (width 0.2) (layer "F.Cu") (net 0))
 (segment (start 143.92 88.92) (end 134.62 79.62) (width 0.2) (layer "F.Cu") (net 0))
 (segment (start 150.568 63.318) (end 161.25 74) (width 0.2) (layer "F.Cu") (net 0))
 (segment (start 175.75 74) (end 175.75 80.925635) (width 0.2) (layer "F.Cu") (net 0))
 (segment (start 143.762944 91.46) (end 144.19 91.46) (width 0.2) (layer "F.Cu") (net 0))
 (segment (start 129.5 68) (end 116.81 68) (width 0.2) (layer "F.Cu") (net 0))
 (segment (start 117.289786 73.478) (end 124.978 73.478) (width 0.2) (layer "F.Cu") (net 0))
 (segment (start 148.561301 109.561301) (end 148.311301 109.811301) (width 0.2) (layer "F.Cu") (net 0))
 (segment (start 155.592157 71.092157) (end 166 81.5) (width 0.2) (layer "F.Cu") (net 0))
 (segment (start 124.978 73.478) (end 128.58 77.08) (width 0.2) (layer "F.Cu") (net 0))
 (segment (start 173.62 78.77) (end 168.85 74) (width 0.2) (layer "F.Cu") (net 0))
 (segment (start 117.705786 65.858) (end 133.558 65.858) (width 0.2) (layer "F.Cu") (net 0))
 (segment (start 149.0075 116.9925) (end 150.54 115.46) (width 0.2) (layer "F.Cu") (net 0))
 (segment (start 131.5 96.5) (end 131.5 99.4125) (width 0.2) (layer "F.Cu") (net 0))
 (segment (start 113.5 65.5) (end 113.5 63.69) (width 0.2) (layer "F.Cu") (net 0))
 (segment (start 114.5 88.39) (end 114.5 76.267786) (width 0.2) (layer "F.Cu") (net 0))
 (segment (start 114.715 62.475) (end 113.5 63.69) (width 0.2) (layer "F.Cu") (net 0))
 (segment (start 161.25 71.5) (end 152.625 62.875) (width 0.2) (layer "F.Cu") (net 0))
 (segment (start 131.5 81.238105) (end 131.5 96.5) (width 0.2) (layer "F.Cu") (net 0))
 (segment (start 134.180105 78.558) (end 131.5 81.238105) (width 0.2) (layer "F.Cu") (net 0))
 (segment (start 154.725 62.475) (end 161.25 69) (width 0.2) (layer "F.Cu") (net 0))
 (segment (start 111 63) (end 111.925 62.075) (width 0.2) (layer "F.Cu") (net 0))
 (segment (start 113 72.5) (end 111 70.5) (width 0.2) (layer "F.Cu") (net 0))
 (segment (start 176 91.5) (end 173.42 88.92) (width 0.2) (layer "F.Cu") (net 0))
 (segment (start 119.38 79.62) (end 130.1 90.34) (width 0.2) (layer "F.Cu") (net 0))
 (segment (start 130.1 90.34) (end 130.1 98.99085) (width 0.2) (layer "F.Cu") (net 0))
 (segment (start 133.953299 103.546701) (end 133.953299 108.147449) (width 0.2) (layer "F.Cu") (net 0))
 (segment (start 152.625 62.875) (end 117.732786 62.875) (width 0.2) (layer "F.Cu") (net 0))
 (segment (start 119.38 77.08) (end 118.30237 77.08) (width 0.2) (layer "F.Cu") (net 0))
 (segment (start 138.722944 96.5) (end 143.762944 91.46) (width 0.2) (layer "F.Cu") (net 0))
 (segment (start 173.62 81.5) (end 173.62 78.77) (width 0.2) (layer "F.Cu") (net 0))
 (segment (start 139.559056 78.558) (end 134.180105 78.558) (width 0.2) (layer "F.Cu") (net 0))
 (segment (start 114.92 66.92) (end 113.5 65.5) (width 0.2) (layer "F.Cu") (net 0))
 (segment (start 165.215635 91.46) (end 164.69 91.46) (width 0.2) (layer "F.Cu") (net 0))
 (segment (start 138.630101 74.54) (end 144.750101 68.42) (width 0.2) (layer "F.Cu") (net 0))
 (segment (start 118.30237 77.08) (end 117 78.38237) (width 0.2) (layer "F.Cu") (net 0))
 (segment (start 142.5 111.39085) (end 142.5 112.392399) (width 0.2) (layer "F.Cu") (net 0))
 (segment (start 133.558 65.858) (end 134.62 66.92) (width 0.2) (layer "F.Cu") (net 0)))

